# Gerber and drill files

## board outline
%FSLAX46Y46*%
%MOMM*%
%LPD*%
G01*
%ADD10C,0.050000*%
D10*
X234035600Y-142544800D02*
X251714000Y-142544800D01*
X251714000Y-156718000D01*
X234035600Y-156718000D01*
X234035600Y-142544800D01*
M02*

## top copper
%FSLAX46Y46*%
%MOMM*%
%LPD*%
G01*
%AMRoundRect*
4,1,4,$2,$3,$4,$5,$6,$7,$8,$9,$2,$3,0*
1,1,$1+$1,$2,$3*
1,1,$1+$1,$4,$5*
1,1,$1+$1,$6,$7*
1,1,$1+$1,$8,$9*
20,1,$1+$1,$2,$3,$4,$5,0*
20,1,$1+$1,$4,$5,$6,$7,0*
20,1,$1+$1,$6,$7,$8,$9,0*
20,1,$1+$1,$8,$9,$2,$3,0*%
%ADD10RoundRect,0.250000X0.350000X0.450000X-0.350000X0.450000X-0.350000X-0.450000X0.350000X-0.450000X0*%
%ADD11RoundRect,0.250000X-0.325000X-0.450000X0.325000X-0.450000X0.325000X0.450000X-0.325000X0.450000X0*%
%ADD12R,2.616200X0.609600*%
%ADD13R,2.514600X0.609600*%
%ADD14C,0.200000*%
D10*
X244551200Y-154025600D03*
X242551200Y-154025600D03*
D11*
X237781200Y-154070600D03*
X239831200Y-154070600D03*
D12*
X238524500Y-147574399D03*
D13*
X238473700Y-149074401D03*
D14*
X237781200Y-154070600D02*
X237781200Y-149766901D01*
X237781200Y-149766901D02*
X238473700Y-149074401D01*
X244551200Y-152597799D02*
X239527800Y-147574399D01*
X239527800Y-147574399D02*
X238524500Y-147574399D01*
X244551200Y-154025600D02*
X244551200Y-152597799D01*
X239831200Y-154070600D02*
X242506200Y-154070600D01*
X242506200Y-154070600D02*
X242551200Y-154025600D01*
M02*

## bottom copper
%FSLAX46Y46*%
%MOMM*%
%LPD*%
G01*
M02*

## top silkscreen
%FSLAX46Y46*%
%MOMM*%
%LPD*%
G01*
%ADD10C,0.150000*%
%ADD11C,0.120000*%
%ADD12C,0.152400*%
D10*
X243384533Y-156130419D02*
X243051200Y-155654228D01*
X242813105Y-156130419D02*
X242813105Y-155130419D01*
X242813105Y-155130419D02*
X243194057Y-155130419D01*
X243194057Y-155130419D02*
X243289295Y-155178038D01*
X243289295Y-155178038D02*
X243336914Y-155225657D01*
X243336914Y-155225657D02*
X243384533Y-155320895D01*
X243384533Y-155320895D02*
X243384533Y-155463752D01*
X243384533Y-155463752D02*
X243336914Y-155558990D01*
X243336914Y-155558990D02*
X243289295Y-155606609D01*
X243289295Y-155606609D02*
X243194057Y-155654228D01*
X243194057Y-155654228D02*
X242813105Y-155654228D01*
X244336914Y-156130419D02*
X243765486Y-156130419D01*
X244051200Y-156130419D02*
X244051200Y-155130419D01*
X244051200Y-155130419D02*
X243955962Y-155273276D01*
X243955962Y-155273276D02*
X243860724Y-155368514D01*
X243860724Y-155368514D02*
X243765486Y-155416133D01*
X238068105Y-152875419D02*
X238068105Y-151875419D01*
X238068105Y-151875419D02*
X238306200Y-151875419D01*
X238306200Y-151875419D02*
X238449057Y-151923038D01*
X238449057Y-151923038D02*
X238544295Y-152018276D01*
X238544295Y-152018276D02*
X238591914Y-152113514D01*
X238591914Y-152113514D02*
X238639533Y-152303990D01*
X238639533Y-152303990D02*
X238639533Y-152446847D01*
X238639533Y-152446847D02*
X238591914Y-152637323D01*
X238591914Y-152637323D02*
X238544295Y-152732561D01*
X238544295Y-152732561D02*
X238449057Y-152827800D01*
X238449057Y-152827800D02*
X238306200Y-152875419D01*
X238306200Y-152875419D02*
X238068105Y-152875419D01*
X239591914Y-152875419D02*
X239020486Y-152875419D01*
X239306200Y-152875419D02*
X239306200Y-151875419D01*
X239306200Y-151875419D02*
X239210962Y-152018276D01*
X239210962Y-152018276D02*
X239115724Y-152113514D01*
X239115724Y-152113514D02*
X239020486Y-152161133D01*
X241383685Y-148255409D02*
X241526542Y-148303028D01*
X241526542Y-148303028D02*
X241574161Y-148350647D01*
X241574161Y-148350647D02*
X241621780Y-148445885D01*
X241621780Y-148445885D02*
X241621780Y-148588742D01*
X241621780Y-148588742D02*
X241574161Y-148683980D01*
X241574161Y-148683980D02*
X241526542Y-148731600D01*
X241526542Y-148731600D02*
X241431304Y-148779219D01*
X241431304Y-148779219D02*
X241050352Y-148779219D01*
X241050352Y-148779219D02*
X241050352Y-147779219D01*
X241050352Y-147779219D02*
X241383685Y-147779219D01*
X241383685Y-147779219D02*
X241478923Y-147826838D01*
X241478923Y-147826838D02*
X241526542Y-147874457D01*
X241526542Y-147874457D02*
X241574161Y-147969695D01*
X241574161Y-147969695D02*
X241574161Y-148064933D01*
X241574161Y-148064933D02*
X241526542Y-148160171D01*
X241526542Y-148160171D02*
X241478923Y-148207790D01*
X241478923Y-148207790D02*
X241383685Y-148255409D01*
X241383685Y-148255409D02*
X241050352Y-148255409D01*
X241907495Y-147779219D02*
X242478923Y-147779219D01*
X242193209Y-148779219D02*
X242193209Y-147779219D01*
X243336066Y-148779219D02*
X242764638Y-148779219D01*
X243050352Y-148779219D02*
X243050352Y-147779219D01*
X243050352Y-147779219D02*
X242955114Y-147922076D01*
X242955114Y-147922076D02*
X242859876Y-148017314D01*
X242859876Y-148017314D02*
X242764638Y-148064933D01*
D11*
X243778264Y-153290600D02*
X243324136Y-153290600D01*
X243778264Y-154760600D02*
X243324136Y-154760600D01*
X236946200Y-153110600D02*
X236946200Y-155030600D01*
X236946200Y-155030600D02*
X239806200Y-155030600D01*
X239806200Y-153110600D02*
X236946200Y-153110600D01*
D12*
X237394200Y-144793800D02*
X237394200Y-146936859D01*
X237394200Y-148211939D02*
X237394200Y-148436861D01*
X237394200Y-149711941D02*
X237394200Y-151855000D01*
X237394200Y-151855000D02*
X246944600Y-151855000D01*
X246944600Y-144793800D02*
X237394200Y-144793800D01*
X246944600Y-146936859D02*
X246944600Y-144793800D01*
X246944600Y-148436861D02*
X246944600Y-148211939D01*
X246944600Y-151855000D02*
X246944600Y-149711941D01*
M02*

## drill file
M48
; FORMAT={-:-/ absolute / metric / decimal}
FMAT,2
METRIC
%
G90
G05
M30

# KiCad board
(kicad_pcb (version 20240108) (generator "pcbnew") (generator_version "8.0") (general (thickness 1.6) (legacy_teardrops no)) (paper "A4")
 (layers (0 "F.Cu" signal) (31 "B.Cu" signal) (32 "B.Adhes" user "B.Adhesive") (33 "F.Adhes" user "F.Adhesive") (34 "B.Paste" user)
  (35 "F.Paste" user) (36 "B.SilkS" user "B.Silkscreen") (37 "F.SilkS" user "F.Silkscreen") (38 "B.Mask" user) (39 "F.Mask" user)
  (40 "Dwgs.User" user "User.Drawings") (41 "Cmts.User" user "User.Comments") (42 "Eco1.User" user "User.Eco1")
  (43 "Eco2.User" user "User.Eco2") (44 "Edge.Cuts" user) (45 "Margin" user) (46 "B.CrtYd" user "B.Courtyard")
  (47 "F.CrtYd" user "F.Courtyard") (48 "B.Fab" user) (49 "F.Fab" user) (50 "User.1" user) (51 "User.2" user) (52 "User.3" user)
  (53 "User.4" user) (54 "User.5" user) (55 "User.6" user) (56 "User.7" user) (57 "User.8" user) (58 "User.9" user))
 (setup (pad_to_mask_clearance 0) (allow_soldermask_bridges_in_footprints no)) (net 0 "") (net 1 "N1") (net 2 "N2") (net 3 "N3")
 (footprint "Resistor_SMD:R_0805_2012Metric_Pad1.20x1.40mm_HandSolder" (layer "F.Cu") (at 243.5512 154.0256 180)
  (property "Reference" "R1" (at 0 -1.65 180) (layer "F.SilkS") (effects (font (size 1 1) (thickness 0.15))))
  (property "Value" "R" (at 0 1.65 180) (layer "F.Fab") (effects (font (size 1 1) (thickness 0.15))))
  (fp_line (start -0.227064 0.735) (end 0.227064 0.735) (stroke (width 0.12) (type solid)) (layer "F.SilkS"))
  (fp_line (start -0.227064 -0.735) (end 0.227064 -0.735) (stroke (width 0.12) (type solid)) (layer "F.SilkS"))
  (pad "1" smd roundrect (at -1 0 180) (size 1.2 1.4) (layers "F.Cu" "F.Paste" "F.Mask") (roundrect_rratio 0.208333) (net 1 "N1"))
  (pad "2" smd roundrect (at 1 0 180) (size 1.2 1.4) (layers "F.Cu" "F.Paste" "F.Mask") (roundrect_rratio 0.208333) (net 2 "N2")))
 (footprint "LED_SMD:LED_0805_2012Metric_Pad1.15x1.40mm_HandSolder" (layer "F.Cu") (at 238.8062 154.0706)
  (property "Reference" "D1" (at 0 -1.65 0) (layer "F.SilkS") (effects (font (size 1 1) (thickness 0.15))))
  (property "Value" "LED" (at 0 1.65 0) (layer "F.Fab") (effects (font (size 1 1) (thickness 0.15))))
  (fp_line (start -1.86 -0.96) (end -1.86 0.96) (stroke (width 0.12) (type solid)) (layer "F.SilkS"))
  (fp_line (start -1.86 0.96) (end 1 0.96) (stroke (width 0.12) (type solid)) (layer "F.SilkS"))
  (fp_line (start 1 -0.96) (end -1.86 -0.96) (stroke (width 0.12) (type solid)) (layer "F.SilkS"))
  (pad "1" smd roundrect (at -1.025 0) (size 1.15 1.4) (layers "F.Cu" "F.Paste" "F.Mask") (roundrect_rratio 0.217391) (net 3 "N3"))
  (pad "2" smd roundrect (at 1.025 0) (size 1.15 1.4) (layers "F.Cu" "F.Paste" "F.Mask") (roundrect_rratio 0.217391) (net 2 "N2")))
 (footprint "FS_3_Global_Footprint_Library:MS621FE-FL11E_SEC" (layer "F.Cu") (at 242.1694 148.3244)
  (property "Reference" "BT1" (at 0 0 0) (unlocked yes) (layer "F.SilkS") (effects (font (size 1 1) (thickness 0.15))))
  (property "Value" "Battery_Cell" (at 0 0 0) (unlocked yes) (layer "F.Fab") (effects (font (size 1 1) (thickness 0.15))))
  (fp_line (start -4.7752 -3.5306) (end -4.7752 -1.387541) (stroke (width 0.1524) (type solid)) (layer "F.SilkS"))
  (fp_line (start -4.7752 -0.112461) (end -4.7752 0.112461) (stroke (width 0.1524) (type solid)) (layer "F.SilkS"))
  (fp_line (start -4.7752 1.387541) (end -4.7752 3.5306) (stroke (width 0.1524) (type solid)) (layer "F.SilkS"))
  (fp_line (start -4.7752 3.5306) (end 4.7752 3.5306) (stroke (width 0.1524) (type solid)) (layer "F.SilkS"))
  (fp_line (start 4.7752 -3.5306) (end -4.7752 -3.5306) (stroke (width 0.1524) (type solid)) (layer "F.SilkS"))
  (fp_line (start 4.7752 -1.387541) (end 4.7752 -3.5306) (stroke (width 0.1524) (type solid)) (layer "F.SilkS"))
  (fp_line (start 4.7752 0.112461) (end 4.7752 -0.112461) (stroke (width 0.1524) (type solid)) (layer "F.SilkS"))
  (fp_line (start 4.7752 3.5306) (end 4.7752 1.387541) (stroke (width 0.1524) (type solid)) (layer "F.SilkS"))
  (pad "1" smd rect (at -3.6449 -0.750001) (size 2.6162 0.6096) (layers "F.Cu" "F.Paste" "F.Mask") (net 1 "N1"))
  (pad "2" smd rect (at -3.6957 0.750001) (size 2.5146 0.6096) (layers "F.Cu" "F.Paste" "F.Mask") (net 3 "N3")))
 (gr_rect (start 234.0356 142.5448) (end 251.714 156.718) (stroke (width 0.05) (type default)) (fill none) (layer "Edge.Cuts"))
 (segment (start 237.7812 154.0706) (end 237.7812 149.766901) (width 0.2) (layer "F.Cu") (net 3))
 (segment (start 237.7812 149.766901) (end 238.4737 149.074401) (width 0.2) (layer "F.Cu") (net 3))
 (segment (start 244.5512 152.597799) (end 239.5278 147.574399) (width 0.2) (layer "F.Cu") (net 1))
 (segment (start 239.5278 147.574399) (end 238.5245 147.574399) (width 0.2) (layer "F.Cu") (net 1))
 (segment (start 244.5512 154.0256) (end 244.5512 152.597799) (width 0.2) (layer "F.Cu") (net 1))
 (segment (start 239.8312 154.0706) (end 242.5062 154.0706) (width 0.2) (layer "F.Cu") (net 2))
 (segment (start 242.5062 154.0706) (end 242.5512 154.0256) (width 0.2) (layer "F.Cu") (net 2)))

